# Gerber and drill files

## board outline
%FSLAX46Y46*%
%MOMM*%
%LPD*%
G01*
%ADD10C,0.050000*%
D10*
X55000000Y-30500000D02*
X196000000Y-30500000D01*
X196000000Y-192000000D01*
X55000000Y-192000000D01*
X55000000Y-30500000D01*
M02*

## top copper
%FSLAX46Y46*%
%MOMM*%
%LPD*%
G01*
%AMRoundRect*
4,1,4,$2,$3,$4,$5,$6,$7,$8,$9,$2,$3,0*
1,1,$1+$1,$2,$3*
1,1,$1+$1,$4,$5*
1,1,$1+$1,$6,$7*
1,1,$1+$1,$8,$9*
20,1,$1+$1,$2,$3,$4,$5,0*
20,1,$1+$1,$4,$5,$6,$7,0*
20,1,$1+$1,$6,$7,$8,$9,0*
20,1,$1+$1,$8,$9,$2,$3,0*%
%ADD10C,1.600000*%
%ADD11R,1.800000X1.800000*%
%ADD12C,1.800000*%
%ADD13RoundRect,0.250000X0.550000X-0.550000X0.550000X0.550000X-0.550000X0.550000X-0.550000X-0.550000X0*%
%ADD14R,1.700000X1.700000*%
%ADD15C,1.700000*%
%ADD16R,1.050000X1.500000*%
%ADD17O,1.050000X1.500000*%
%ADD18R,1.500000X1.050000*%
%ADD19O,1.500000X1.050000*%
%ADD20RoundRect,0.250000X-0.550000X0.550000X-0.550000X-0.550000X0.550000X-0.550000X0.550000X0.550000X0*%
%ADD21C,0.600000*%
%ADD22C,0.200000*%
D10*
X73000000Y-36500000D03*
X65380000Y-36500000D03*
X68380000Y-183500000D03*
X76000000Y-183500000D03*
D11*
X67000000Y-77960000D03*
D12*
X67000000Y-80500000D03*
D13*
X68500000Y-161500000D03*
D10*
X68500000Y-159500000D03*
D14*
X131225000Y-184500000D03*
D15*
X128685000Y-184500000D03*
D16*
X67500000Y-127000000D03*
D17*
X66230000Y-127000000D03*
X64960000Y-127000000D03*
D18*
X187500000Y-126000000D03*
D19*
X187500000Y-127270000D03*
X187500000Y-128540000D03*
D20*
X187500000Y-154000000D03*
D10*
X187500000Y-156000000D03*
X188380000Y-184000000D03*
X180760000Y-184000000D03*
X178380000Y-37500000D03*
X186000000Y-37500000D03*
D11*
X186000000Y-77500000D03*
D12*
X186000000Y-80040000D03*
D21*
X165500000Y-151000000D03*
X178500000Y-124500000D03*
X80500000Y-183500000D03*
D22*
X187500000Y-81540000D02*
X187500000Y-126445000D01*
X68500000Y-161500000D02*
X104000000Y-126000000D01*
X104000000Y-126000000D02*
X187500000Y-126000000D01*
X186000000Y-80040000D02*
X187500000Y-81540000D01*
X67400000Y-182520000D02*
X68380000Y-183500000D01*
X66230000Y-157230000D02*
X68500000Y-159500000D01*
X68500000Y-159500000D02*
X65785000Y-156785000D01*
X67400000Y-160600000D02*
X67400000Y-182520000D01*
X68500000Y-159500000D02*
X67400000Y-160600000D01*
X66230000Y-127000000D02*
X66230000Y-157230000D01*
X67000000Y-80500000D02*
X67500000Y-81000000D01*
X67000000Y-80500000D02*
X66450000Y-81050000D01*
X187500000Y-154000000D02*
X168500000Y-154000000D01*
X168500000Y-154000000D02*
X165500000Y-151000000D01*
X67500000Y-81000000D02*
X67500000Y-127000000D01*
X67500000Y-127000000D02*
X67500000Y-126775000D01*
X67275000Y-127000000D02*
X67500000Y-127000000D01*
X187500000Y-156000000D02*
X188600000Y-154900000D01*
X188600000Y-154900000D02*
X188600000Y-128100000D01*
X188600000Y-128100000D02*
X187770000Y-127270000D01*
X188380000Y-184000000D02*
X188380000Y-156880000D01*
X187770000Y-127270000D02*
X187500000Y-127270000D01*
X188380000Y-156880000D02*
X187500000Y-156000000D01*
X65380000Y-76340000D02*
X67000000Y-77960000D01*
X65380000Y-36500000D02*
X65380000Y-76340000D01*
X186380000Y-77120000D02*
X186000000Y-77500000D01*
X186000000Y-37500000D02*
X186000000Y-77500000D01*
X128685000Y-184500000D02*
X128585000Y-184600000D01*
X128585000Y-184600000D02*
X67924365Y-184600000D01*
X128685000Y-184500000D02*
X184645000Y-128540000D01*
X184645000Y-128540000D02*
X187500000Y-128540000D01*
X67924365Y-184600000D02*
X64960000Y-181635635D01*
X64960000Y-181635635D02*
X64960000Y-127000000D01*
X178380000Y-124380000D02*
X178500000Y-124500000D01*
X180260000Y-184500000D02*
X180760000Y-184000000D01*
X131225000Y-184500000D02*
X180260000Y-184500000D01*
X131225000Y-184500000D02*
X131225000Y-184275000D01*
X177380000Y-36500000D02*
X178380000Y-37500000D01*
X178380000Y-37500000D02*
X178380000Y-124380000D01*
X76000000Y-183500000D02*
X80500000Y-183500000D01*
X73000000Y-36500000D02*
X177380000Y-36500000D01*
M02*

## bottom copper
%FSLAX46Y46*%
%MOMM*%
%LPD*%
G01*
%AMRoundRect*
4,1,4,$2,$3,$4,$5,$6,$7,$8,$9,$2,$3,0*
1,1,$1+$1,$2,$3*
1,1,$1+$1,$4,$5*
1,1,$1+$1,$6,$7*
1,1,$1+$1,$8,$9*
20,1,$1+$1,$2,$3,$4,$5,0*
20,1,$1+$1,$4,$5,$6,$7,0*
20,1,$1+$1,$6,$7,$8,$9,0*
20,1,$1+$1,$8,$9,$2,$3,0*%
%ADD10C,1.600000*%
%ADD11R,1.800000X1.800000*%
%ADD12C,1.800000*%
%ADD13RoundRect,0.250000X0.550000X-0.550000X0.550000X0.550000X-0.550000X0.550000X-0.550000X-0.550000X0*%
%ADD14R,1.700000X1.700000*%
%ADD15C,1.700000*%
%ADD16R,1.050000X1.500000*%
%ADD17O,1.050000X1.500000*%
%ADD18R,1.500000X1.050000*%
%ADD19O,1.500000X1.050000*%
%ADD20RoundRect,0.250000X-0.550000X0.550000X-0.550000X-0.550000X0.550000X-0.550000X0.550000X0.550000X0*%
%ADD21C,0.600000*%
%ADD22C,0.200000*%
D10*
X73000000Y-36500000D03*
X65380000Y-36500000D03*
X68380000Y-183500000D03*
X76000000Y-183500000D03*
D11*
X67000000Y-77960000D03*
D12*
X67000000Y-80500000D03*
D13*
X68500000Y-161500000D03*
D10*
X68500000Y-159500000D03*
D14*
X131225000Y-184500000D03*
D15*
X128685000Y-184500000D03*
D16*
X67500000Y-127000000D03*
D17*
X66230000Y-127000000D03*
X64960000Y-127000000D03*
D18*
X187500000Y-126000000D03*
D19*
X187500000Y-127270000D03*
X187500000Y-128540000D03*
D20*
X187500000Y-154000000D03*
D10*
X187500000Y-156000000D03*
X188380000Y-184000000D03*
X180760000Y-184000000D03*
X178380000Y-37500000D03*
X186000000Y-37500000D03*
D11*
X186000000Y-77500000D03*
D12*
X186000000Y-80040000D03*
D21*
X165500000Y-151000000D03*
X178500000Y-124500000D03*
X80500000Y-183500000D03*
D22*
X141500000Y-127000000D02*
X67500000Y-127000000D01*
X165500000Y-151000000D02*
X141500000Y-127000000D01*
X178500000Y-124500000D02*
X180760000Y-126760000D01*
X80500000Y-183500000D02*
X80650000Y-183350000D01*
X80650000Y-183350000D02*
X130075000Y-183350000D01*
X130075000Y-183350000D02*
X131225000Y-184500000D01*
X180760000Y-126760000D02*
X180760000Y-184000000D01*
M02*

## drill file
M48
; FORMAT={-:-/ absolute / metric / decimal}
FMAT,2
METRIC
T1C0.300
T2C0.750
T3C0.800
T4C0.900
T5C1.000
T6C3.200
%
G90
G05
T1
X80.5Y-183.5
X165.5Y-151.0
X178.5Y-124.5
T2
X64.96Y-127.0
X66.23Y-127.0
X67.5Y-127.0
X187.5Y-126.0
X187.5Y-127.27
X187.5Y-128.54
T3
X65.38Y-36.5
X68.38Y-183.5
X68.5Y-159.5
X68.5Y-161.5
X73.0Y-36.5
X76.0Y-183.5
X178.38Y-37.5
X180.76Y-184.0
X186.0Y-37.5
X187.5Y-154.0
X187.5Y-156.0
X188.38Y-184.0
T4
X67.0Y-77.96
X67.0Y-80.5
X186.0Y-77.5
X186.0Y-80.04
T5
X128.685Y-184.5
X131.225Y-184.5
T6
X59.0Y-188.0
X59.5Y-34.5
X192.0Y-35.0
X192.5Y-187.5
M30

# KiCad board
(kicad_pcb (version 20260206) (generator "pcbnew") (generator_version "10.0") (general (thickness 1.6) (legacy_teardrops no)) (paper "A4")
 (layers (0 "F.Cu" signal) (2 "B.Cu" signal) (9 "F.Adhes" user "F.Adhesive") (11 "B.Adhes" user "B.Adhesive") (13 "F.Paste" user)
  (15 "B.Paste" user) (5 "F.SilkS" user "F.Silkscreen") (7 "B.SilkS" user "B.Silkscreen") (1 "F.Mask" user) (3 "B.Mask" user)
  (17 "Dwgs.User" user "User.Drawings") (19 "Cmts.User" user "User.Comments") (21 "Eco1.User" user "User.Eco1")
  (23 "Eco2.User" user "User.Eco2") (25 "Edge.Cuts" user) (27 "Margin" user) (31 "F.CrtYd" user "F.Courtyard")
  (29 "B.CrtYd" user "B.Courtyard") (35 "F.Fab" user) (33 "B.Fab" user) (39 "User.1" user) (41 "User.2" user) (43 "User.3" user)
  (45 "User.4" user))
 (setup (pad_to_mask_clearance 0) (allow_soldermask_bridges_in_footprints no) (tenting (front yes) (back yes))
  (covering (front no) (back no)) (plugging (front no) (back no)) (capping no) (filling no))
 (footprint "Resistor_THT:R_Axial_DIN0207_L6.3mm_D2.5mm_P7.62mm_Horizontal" (layer "F.Cu") (at 73 36.5 180)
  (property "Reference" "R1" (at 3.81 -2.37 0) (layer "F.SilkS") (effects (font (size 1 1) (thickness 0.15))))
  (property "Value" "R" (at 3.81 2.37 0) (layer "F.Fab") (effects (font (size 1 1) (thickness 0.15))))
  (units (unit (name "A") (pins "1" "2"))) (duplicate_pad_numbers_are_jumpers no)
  (pad "1" thru_hole circle (at 0 0 180) (size 1.6 1.6) (drill 0.8) (layers "*.Cu" "*.Mask") (remove_unused_layers no) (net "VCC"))
  (pad "2" thru_hole circle (at 7.62 0 180) (size 1.6 1.6) (drill 0.8) (layers "*.Cu" "*.Mask") (remove_unused_layers no) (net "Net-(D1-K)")))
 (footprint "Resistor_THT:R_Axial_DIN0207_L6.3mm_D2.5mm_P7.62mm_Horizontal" (layer "F.Cu") (at 68.38 183.5)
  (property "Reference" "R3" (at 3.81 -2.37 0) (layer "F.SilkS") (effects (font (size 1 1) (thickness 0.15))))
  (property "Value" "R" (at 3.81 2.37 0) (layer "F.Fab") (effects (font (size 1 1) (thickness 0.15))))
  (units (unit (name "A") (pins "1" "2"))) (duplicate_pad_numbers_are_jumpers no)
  (pad "1" thru_hole circle (at 0 0) (size 1.6 1.6) (drill 0.8) (layers "*.Cu" "*.Mask") (remove_unused_layers no) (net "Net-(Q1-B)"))
  (pad "2" thru_hole circle (at 7.62 0) (size 1.6 1.6) (drill 0.8) (layers "*.Cu" "*.Mask") (remove_unused_layers no) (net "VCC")))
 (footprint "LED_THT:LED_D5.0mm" (layer "F.Cu") (at 67 77.96 -90)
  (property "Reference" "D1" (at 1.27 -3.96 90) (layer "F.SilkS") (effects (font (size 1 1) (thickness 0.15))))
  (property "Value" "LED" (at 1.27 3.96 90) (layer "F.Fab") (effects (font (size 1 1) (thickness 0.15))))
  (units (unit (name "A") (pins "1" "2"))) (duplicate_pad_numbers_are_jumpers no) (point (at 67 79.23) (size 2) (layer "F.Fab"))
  (pad "1" thru_hole rect (at 0 0 270) (size 1.8 1.8) (drill 0.9) (layers "*.Cu" "*.Mask") (remove_unused_layers no) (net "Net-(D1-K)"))
  (pad "2" thru_hole circle (at 2.54 0 270) (size 1.8 1.8) (drill 0.9) (layers "*.Cu" "*.Mask") (remove_unused_layers no) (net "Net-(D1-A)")))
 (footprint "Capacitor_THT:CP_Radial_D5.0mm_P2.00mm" (layer "F.Cu") (at 68.5 161.5 90)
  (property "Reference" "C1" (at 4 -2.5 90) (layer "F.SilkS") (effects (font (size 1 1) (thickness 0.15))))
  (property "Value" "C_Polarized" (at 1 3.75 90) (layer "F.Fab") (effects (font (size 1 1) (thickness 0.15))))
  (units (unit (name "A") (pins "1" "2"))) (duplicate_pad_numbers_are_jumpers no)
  (pad "1" thru_hole roundrect (at 0 0 90) (size 1.6 1.6) (drill 0.8) (layers "*.Cu" "*.Mask") (remove_unused_layers no)
   (roundrect_rratio 0.15625) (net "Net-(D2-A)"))
  (pad "2" thru_hole circle (at 2 0 90) (size 1.6 1.6) (drill 0.8) (layers "*.Cu" "*.Mask") (remove_unused_layers no) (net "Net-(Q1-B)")))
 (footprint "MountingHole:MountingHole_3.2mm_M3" (layer "F.Cu") (at 59 188)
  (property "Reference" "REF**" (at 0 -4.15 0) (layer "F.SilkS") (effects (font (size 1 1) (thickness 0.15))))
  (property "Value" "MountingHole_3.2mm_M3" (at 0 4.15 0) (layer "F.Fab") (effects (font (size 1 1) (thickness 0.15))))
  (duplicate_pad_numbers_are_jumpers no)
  (pad "" np_thru_hole circle (at 0 0) (size 3.2 3.2) (drill 3.2) (layers "*.Cu" "*.Mask")))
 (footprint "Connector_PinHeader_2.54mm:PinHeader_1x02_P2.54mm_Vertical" (layer "F.Cu") (at 131.225 184.5 -90)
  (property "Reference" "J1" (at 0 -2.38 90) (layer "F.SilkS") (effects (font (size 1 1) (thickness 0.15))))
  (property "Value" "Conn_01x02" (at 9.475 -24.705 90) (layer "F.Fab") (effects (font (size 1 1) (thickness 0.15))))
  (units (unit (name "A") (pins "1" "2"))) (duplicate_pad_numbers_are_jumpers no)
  (pad "1" thru_hole rect (at 0 0 270) (size 1.7 1.7) (drill 1) (layers "*.Cu" "*.Mask") (remove_unused_layers no) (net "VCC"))
  (pad "2" thru_hole circle (at 0 2.54 270) (size 1.7 1.7) (drill 1) (layers "*.Cu" "*.Mask") (remove_unused_layers no) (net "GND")))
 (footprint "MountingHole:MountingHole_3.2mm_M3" (layer "F.Cu") (at 192.5 187.5)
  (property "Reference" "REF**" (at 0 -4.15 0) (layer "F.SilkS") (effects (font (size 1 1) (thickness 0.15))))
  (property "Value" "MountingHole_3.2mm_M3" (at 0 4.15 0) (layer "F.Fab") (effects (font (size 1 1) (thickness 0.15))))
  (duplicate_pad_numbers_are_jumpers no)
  (pad "" np_thru_hole circle (at 0 0) (size 3.2 3.2) (drill 3.2) (layers "*.Cu" "*.Mask")))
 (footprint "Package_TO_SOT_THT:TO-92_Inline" (layer "F.Cu") (at 67.5 127 180)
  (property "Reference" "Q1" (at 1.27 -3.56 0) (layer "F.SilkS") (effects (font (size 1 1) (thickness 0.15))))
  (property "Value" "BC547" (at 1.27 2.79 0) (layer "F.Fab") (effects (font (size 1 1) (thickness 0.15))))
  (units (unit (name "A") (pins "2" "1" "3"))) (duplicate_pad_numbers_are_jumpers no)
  (pad "1" thru_hole rect (at 0 0 180) (size 1.05 1.5) (drill 0.75) (layers "*.Cu" "*.Mask") (remove_unused_layers no) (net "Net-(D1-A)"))
  (pad "2" thru_hole oval (at 1.27 0 180) (size 1.05 1.5) (drill 0.75) (layers "*.Cu" "*.Mask") (remove_unused_layers no) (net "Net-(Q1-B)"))
  (pad "3" thru_hole oval (at 2.54 0 180) (size 1.05 1.5) (drill 0.75) (layers "*.Cu" "*.Mask") (remove_unused_layers no) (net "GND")))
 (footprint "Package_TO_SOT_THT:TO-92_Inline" (layer "F.Cu") (at 187.5 126 -90)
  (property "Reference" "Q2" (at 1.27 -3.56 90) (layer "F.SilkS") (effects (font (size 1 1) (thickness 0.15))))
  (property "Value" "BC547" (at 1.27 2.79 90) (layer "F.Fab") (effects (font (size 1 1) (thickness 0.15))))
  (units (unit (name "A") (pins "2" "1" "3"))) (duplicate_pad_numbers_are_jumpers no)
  (pad "1" thru_hole rect (at 0 0 270) (size 1.05 1.5) (drill 0.75) (layers "*.Cu" "*.Mask") (remove_unused_layers no) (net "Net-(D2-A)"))
  (pad "2" thru_hole oval (at 1.27 0 270) (size 1.05 1.5) (drill 0.75) (layers "*.Cu" "*.Mask") (remove_unused_layers no) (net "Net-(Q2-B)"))
  (pad "3" thru_hole oval (at 2.54 0 270) (size 1.05 1.5) (drill 0.75) (layers "*.Cu" "*.Mask") (remove_unused_layers no) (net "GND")))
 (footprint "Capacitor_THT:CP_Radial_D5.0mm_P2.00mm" (layer "F.Cu") (at 187.5 154 -90)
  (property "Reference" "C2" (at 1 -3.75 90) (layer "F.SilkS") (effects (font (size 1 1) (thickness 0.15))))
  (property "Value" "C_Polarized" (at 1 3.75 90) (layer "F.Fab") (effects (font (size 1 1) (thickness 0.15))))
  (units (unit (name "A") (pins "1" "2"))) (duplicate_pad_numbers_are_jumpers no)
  (pad "1" thru_hole roundrect (at 0 0 270) (size 1.6 1.6) (drill 0.8) (layers "*.Cu" "*.Mask") (remove_unused_layers no)
   (roundrect_rratio 0.15625) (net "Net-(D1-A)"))
  (pad "2" thru_hole circle (at 2 0 270) (size 1.6 1.6) (drill 0.8) (layers "*.Cu" "*.Mask") (remove_unused_layers no) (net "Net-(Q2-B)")))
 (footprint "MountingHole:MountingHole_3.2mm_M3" (layer "F.Cu") (at 192 35)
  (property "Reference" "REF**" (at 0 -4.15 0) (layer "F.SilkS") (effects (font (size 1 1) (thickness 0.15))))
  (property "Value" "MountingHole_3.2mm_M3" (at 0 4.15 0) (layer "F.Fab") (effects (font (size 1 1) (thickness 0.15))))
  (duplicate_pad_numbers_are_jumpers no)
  (pad "" np_thru_hole circle (at 0 0) (size 3.2 3.2) (drill 3.2) (layers "*.Cu" "*.Mask")))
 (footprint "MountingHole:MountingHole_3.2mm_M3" (layer "F.Cu") (at 59.5 34.5)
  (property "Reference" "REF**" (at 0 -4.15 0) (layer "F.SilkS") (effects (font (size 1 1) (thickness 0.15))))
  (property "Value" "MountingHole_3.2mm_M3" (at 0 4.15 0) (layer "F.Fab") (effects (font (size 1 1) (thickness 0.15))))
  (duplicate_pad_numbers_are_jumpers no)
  (pad "" np_thru_hole circle (at 0 0) (size 3.2 3.2) (drill 3.2) (layers "*.Cu" "*.Mask")))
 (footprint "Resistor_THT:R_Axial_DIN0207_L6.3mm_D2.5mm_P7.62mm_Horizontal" (layer "F.Cu") (at 188.38 184 180)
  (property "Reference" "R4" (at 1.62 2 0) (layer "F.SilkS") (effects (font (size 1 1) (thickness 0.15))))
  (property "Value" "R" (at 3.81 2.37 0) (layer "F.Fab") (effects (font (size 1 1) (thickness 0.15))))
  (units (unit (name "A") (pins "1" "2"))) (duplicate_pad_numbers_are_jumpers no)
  (pad "1" thru_hole circle (at 0 0 180) (size 1.6 1.6) (drill 0.8) (layers "*.Cu" "*.Mask") (remove_unused_layers no) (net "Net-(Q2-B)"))
  (pad "2" thru_hole circle (at 7.62 0 180) (size 1.6 1.6) (drill 0.8) (layers "*.Cu" "*.Mask") (remove_unused_layers no) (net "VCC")))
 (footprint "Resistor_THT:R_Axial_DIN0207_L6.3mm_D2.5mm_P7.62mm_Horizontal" (layer "F.Cu") (at 178.38 37.5)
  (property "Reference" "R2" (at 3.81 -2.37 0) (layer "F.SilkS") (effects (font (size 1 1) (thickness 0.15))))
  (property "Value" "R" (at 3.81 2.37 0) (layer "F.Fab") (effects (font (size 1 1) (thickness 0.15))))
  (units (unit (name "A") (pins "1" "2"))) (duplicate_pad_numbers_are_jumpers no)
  (pad "1" thru_hole circle (at 0 0) (size 1.6 1.6) (drill 0.8) (layers "*.Cu" "*.Mask") (remove_unused_layers no) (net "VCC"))
  (pad "2" thru_hole circle (at 7.62 0) (size 1.6 1.6) (drill 0.8) (layers "*.Cu" "*.Mask") (remove_unused_layers no) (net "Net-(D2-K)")))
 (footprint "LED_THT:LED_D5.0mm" (layer "F.Cu") (at 186 77.5 -90)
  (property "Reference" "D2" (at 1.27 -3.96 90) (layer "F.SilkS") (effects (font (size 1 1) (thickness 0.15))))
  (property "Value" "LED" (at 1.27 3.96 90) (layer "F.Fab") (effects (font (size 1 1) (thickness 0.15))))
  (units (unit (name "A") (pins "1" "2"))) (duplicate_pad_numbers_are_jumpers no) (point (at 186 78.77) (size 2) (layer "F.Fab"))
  (pad "1" thru_hole rect (at 0 0 270) (size 1.8 1.8) (drill 0.9) (layers "*.Cu" "*.Mask") (remove_unused_layers no) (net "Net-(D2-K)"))
  (pad "2" thru_hole circle (at 2.54 0 270) (size 1.8 1.8) (drill 0.9) (layers "*.Cu" "*.Mask") (remove_unused_layers no) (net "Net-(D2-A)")))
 (gr_rect (start 55 30.5) (end 196 192) (stroke (width 0.05) (type default)) (fill no) (layer "Edge.Cuts"))
 (segment (start 187.5 81.54) (end 187.5 126.445) (width 0.2) (layer "F.Cu") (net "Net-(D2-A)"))
 (segment (start 68.5 161.5) (end 104 126) (width 0.2) (layer "F.Cu") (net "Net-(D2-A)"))
 (segment (start 104 126) (end 187.5 126) (width 0.2) (layer "F.Cu") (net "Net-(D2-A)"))
 (segment (start 186 80.04) (end 187.5 81.54) (width 0.2) (layer "F.Cu") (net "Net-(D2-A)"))
 (segment (start 67.4 182.52) (end 68.38 183.5) (width 0.2) (layer "F.Cu") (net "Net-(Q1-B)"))
 (segment (start 66.23 157.23) (end 68.5 159.5) (width 0.2) (layer "F.Cu") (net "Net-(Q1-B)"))
 (segment (start 68.5 159.5) (end 65.785 156.785) (width 0.2) (layer "F.Cu") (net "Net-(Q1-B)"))
 (segment (start 67.4 160.6) (end 67.4 182.52) (width 0.2) (layer "F.Cu") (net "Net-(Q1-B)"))
 (segment (start 68.5 159.5) (end 67.4 160.6) (width 0.2) (layer "F.Cu") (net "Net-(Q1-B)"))
 (segment (start 66.23 127) (end 66.23 157.23) (width 0.2) (layer "F.Cu") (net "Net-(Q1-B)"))
 (segment (start 67 80.5) (end 67.5 81) (width 0.2) (layer "F.Cu") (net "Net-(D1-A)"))
 (segment (start 67 80.5) (end 66.45 81.05) (width 0.2) (layer "F.Cu") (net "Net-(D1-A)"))
 (segment (start 187.5 154) (end 168.5 154) (width 0.2) (layer "F.Cu") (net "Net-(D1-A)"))
 (segment (start 168.5 154) (end 165.5 151) (width 0.2) (layer "F.Cu") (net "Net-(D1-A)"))
 (segment (start 67.5 81) (end 67.5 127) (width 0.2) (layer "F.Cu") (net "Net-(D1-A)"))
 (segment (start 67.5 127) (end 67.5 126.775) (width 0.2) (layer "F.Cu") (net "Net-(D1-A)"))
 (segment (start 67.275 127) (end 67.5 127) (width 0.2) (layer "F.Cu") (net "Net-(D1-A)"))
 (via (at 165.5 151) (size 0.6) (drill 0.3) (layers "F.Cu" "B.Cu") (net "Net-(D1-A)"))
 (segment (start 141.5 127) (end 67.5 127) (width 0.2) (layer "B.Cu") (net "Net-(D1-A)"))
 (segment (start 165.5 151) (end 141.5 127) (width 0.2) (layer "B.Cu") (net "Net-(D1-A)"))
 (segment (start 187.5 156) (end 188.6 154.9) (width 0.2) (layer "F.Cu") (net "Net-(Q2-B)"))
 (segment (start 188.6 154.9) (end 188.6 128.1) (width 0.2) (layer "F.Cu") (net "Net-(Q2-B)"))
 (segment (start 188.6 128.1) (end 187.77 127.27) (width 0.2) (layer "F.Cu") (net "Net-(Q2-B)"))
 (segment (start 188.38 184) (end 188.38 156.88) (width 0.2) (layer "F.Cu") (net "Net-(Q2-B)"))
 (segment (start 187.77 127.27) (end 187.5 127.27) (width 0.2) (layer "F.Cu") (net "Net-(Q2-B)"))
 (segment (start 188.38 156.88) (end 187.5 156) (width 0.2) (layer "F.Cu") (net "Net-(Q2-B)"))
 (segment (start 65.38 76.34) (end 67 77.96) (width 0.2) (layer "F.Cu") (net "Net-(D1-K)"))
 (segment (start 65.38 36.5) (end 65.38 76.34) (width 0.2) (layer "F.Cu") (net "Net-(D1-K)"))
 (segment (start 186.38 77.12) (end 186 77.5) (width 0.2) (layer "F.Cu") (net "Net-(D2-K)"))
 (segment (start 186 37.5) (end 186 77.5) (width 0.2) (layer "F.Cu") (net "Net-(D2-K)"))
 (segment (start 128.685 184.5) (end 128.585 184.6) (width 0.2) (layer "F.Cu") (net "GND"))
 (segment (start 128.585 184.6) (end 67.924365 184.6) (width 0.2) (layer "F.Cu") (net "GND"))
 (segment (start 128.685 184.5) (end 184.645 128.54) (width 0.2) (layer "F.Cu") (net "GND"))
 (segment (start 184.645 128.54) (end 187.5 128.54) (width 0.2) (layer "F.Cu") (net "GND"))
 (segment (start 67.924365 184.6) (end 64.96 181.635635) (width 0.2) (layer "F.Cu") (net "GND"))
 (segment (start 64.96 181.635635) (end 64.96 127) (width 0.2) (layer "F.Cu") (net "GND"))
 (segment (start 178.38 124.38) (end 178.5 124.5) (width 0.2) (layer "F.Cu") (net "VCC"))
 (segment (start 180.26 184.5) (end 180.76 184) (width 0.2) (layer "F.Cu") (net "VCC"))
 (segment (start 131.225 184.5) (end 180.26 184.5) (width 0.2) (layer "F.Cu") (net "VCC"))
 (segment (start 131.225 184.5) (end 131.225 184.275) (width 0.2) (layer "F.Cu") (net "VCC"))
 (segment (start 177.38 36.5) (end 178.38 37.5) (width 0.2) (layer "F.Cu") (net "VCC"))
 (segment (start 178.38 37.5) (end 178.38 124.38) (width 0.2) (layer "F.Cu") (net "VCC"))
 (segment (start 76 183.5) (end 80.5 183.5) (width 0.2) (layer "F.Cu") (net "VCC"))
 (segment (start 73 36.5) (end 177.38 36.5) (width 0.2) (layer "F.Cu") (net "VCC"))
 (via (at 178.5 124.5) (size 0.6) (drill 0.3) (layers "F.Cu" "B.Cu") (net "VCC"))
 (via (at 80.5 183.5) (size 0.6) (drill 0.3) (layers "F.Cu" "B.Cu") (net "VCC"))
 (segment (start 178.5 124.5) (end 180.76 126.76) (width 0.2) (layer "B.Cu") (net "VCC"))
 (segment (start 80.5 183.5) (end 80.65 183.35) (width 0.2) (layer "B.Cu") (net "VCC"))
 (segment (start 80.65 183.35) (end 130.075 183.35) (width 0.2) (layer "B.Cu") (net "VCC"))
 (segment (start 130.075 183.35) (end 131.225 184.5) (width 0.2) (layer "B.Cu") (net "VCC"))
 (segment (start 180.76 126.76) (end 180.76 184) (width 0.2) (layer "B.Cu") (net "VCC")))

